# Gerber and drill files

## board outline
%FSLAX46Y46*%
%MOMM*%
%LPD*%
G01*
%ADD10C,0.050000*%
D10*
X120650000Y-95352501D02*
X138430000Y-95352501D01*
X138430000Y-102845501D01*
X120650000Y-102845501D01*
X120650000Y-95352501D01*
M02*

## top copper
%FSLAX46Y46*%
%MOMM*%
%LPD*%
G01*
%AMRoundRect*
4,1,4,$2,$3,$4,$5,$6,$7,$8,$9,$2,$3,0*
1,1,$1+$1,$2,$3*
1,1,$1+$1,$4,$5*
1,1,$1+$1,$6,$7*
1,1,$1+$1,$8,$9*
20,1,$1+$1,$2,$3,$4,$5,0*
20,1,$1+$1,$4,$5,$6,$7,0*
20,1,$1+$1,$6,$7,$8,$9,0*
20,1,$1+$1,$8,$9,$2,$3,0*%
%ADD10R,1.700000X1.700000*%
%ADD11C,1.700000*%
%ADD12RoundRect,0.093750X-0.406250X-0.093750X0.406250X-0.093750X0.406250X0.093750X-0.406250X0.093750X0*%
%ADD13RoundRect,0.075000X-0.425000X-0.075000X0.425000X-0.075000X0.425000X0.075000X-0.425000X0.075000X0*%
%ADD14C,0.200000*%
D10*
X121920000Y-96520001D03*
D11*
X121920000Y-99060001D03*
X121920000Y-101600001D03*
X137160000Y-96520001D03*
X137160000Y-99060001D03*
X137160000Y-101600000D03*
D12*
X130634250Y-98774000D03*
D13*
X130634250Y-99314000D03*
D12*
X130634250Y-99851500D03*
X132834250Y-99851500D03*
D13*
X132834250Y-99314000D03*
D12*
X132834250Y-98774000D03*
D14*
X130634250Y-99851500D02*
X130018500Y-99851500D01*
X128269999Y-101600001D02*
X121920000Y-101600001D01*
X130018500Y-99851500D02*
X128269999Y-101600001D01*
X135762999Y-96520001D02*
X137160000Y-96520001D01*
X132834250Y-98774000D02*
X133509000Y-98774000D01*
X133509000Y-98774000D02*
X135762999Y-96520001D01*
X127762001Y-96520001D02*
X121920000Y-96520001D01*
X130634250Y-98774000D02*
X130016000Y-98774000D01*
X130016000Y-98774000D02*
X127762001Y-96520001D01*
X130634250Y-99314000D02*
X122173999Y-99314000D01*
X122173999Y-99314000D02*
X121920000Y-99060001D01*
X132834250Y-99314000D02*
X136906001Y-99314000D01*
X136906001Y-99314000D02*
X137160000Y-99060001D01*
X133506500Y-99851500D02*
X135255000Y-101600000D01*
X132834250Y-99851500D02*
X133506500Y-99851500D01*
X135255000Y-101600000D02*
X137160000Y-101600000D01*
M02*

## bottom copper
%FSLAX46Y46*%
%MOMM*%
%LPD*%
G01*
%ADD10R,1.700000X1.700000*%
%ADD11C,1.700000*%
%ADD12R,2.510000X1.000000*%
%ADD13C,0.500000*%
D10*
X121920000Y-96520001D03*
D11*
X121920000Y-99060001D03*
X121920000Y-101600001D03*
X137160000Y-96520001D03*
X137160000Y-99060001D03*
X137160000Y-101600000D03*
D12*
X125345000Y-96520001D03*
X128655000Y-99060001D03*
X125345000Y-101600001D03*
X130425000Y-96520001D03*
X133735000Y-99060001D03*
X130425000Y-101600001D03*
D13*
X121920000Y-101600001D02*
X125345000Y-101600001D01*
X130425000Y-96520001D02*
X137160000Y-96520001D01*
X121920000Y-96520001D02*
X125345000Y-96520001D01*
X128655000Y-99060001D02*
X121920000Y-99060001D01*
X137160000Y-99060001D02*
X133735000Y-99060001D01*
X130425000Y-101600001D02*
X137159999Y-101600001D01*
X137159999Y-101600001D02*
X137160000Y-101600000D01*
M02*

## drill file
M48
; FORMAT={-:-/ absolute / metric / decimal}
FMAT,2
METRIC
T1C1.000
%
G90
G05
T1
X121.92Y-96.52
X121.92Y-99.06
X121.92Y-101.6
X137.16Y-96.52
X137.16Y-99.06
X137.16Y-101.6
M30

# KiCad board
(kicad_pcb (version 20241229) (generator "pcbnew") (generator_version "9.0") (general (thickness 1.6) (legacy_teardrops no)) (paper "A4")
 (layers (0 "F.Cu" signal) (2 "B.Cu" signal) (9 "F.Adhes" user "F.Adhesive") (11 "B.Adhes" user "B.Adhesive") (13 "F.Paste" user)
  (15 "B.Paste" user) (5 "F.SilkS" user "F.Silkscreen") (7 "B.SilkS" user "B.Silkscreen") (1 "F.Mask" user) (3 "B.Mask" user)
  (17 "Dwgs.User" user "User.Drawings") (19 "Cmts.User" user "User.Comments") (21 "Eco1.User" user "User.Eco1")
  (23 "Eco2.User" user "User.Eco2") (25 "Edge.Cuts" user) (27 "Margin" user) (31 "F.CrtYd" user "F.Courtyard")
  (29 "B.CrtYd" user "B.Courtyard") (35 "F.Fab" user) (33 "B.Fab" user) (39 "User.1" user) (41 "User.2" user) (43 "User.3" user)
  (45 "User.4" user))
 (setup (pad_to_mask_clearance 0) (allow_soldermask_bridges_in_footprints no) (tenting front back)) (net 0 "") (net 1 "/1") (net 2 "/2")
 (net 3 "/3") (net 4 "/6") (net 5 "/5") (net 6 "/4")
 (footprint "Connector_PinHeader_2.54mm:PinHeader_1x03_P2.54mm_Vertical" (layer "F.Cu") (at 121.92 96.520001)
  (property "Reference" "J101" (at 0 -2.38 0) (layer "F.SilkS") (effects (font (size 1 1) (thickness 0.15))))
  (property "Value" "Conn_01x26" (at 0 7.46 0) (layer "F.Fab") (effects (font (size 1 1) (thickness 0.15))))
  (pad "1" thru_hole rect (at 0 0) (size 1.7 1.7) (drill 1) (layers "*.Cu" "*.Mask") (remove_unused_layers no) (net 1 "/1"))
  (pad "2" thru_hole circle (at 0 2.54) (size 1.7 1.7) (drill 1) (layers "*.Cu" "*.Mask") (remove_unused_layers no) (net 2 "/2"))
  (pad "3" thru_hole circle (at 0 5.08) (size 1.7 1.7) (drill 1) (layers "*.Cu" "*.Mask") (remove_unused_layers no) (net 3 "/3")))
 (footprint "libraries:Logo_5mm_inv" (layer "F.Cu") (at 131.73425 96.774)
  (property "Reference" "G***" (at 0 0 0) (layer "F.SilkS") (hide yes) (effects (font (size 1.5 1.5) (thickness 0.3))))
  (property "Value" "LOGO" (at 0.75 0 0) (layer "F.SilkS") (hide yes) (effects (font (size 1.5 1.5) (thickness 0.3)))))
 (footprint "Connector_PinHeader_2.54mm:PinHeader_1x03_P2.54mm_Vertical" (layer "F.Cu") (at 137.16 96.520001)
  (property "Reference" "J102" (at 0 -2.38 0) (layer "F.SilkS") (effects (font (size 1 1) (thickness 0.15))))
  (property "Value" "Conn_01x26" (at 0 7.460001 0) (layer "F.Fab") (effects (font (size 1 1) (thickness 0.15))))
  (pad "1" thru_hole circle (at 0 0) (size 1.7 1.7) (drill 1) (layers "*.Cu" "*.Mask") (remove_unused_layers no) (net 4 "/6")
   (thermal_bridge_angle 90))
  (pad "2" thru_hole circle (at 0 2.54) (size 1.7 1.7) (drill 1) (layers "*.Cu" "*.Mask") (remove_unused_layers no) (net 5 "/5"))
  (pad "3" thru_hole circle (at 0 5.079999) (size 1.7 1.7) (drill 1) (layers "*.Cu" "*.Mask") (remove_unused_layers no) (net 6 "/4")))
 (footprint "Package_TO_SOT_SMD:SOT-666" (layer "F.Cu") (at 131.73425 99.314)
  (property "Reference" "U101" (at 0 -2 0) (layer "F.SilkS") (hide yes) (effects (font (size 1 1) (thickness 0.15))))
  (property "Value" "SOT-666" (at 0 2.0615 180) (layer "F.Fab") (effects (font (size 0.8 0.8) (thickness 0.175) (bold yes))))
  (pad "1" smd roundrect (at -1.1 -0.54) (size 1 0.375) (layers "F.Cu" "F.Mask" "F.Paste") (roundrect_rratio 0.25) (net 1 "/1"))
  (pad "2" smd roundrect (at -1.1 0) (size 1 0.3) (layers "F.Cu" "F.Mask" "F.Paste") (roundrect_rratio 0.25) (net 2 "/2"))
  (pad "3" smd roundrect (at -1.1 0.5375) (size 1 0.375) (layers "F.Cu" "F.Mask" "F.Paste") (roundrect_rratio 0.25) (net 3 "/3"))
  (pad "4" smd roundrect (at 1.1 0.5375) (size 1 0.375) (layers "F.Cu" "F.Mask" "F.Paste") (roundrect_rratio 0.25) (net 6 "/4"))
  (pad "5" smd roundrect (at 1.1 0) (size 1 0.3) (layers "F.Cu" "F.Mask" "F.Paste") (roundrect_rratio 0.25) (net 5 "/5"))
  (pad "6" smd roundrect (at 1.1 -0.54) (size 1 0.375) (layers "F.Cu" "F.Mask" "F.Paste") (roundrect_rratio 0.25) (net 4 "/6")))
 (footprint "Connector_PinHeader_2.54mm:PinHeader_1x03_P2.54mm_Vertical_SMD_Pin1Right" (layer "B.Cu") (at 127 99.060001 180)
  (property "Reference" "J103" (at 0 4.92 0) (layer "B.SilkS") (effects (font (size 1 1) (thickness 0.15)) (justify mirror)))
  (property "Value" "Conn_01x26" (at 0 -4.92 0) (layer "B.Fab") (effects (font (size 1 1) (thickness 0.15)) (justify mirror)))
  (pad "1" smd rect (at 1.655 2.54 180) (size 2.51 1) (layers "B.Cu" "B.Mask" "B.Paste") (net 1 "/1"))
  (pad "2" smd rect (at -1.655 0 180) (size 2.51 1) (layers "B.Cu" "B.Mask" "B.Paste") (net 2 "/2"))
  (pad "3" smd rect (at 1.655 -2.54 180) (size 2.51 1) (layers "B.Cu" "B.Mask" "B.Paste") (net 3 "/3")))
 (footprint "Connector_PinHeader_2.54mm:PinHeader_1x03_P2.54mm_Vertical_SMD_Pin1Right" (layer "B.Cu") (at 132.08 99.060001 180)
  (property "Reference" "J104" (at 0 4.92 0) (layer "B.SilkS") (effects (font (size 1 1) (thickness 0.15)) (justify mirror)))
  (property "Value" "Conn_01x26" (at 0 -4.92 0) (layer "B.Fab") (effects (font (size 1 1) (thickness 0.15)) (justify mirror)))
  (pad "1" smd rect (at 1.655 2.54 180) (size 2.51 1) (layers "B.Cu" "B.Mask" "B.Paste") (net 4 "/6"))
  (pad "2" smd rect (at -1.655 0 180) (size 2.51 1) (layers "B.Cu" "B.Mask" "B.Paste") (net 5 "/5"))
  (pad "3" smd rect (at 1.655 -2.54 180) (size 2.51 1) (layers "B.Cu" "B.Mask" "B.Paste") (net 6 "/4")))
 (gr_rect (start 120.65 95.352501) (end 138.43 102.845501) (stroke (width 0.05) (type default)) (fill no) (layer "Edge.Cuts"))
 (segment (start 130.63425 99.8515) (end 130.0185 99.8515) (width 0.2) (layer "F.Cu") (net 3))
 (segment (start 128.269999 101.600001) (end 121.92 101.600001) (width 0.2) (layer "F.Cu") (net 3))
 (segment (start 130.0185 99.8515) (end 128.269999 101.600001) (width 0.2) (layer "F.Cu") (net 3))
 (segment (start 121.92 101.600001) (end 125.345 101.600001) (width 0.5) (layer "B.Cu") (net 3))
 (segment (start 135.762999 96.520001) (end 137.16 96.520001) (width 0.2) (layer "F.Cu") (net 4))
 (segment (start 132.83425 98.774) (end 133.509 98.774) (width 0.2) (layer "F.Cu") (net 4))
 (segment (start 133.509 98.774) (end 135.762999 96.520001) (width 0.2) (layer "F.Cu") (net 4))
 (segment (start 130.425 96.520001) (end 137.16 96.520001) (width 0.5) (layer "B.Cu") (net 4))
 (segment (start 127.762001 96.520001) (end 121.92 96.520001) (width 0.2) (layer "F.Cu") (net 1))
 (segment (start 130.63425 98.774) (end 130.016 98.774) (width 0.2) (layer "F.Cu") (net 1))
 (segment (start 130.016 98.774) (end 127.762001 96.520001) (width 0.2) (layer "F.Cu") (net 1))
 (segment (start 121.92 96.520001) (end 125.345 96.520001) (width 0.5) (layer "B.Cu") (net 1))
 (segment (start 130.63425 99.314) (end 122.173999 99.314) (width 0.2) (layer "F.Cu") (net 2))
 (segment (start 122.173999 99.314) (end 121.92 99.060001) (width 0.2) (layer "F.Cu") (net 2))
 (segment (start 128.655 99.060001) (end 121.92 99.060001) (width 0.5) (layer "B.Cu") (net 2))
 (segment (start 132.83425 99.314) (end 136.906001 99.314) (width 0.2) (layer "F.Cu") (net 5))
 (segment (start 136.906001 99.314) (end 137.16 99.060001) (width 0.2) (layer "F.Cu") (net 5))
 (segment (start 137.16 99.060001) (end 133.735 99.060001) (width 0.5) (layer "B.Cu") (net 5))
 (segment (start 133.5065 99.8515) (end 135.255 101.6) (width 0.2) (layer "F.Cu") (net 6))
 (segment (start 132.83425 99.8515) (end 133.5065 99.8515) (width 0.2) (layer "F.Cu") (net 6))
 (segment (start 135.255 101.6) (end 137.16 101.6) (width 0.2) (layer "F.Cu") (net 6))
 (segment (start 130.425 101.600001) (end 137.159999 101.600001) (width 0.5) (layer "B.Cu") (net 6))
 (segment (start 137.159999 101.600001) (end 137.16 101.6) (width 0.5) (layer "B.Cu") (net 6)))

